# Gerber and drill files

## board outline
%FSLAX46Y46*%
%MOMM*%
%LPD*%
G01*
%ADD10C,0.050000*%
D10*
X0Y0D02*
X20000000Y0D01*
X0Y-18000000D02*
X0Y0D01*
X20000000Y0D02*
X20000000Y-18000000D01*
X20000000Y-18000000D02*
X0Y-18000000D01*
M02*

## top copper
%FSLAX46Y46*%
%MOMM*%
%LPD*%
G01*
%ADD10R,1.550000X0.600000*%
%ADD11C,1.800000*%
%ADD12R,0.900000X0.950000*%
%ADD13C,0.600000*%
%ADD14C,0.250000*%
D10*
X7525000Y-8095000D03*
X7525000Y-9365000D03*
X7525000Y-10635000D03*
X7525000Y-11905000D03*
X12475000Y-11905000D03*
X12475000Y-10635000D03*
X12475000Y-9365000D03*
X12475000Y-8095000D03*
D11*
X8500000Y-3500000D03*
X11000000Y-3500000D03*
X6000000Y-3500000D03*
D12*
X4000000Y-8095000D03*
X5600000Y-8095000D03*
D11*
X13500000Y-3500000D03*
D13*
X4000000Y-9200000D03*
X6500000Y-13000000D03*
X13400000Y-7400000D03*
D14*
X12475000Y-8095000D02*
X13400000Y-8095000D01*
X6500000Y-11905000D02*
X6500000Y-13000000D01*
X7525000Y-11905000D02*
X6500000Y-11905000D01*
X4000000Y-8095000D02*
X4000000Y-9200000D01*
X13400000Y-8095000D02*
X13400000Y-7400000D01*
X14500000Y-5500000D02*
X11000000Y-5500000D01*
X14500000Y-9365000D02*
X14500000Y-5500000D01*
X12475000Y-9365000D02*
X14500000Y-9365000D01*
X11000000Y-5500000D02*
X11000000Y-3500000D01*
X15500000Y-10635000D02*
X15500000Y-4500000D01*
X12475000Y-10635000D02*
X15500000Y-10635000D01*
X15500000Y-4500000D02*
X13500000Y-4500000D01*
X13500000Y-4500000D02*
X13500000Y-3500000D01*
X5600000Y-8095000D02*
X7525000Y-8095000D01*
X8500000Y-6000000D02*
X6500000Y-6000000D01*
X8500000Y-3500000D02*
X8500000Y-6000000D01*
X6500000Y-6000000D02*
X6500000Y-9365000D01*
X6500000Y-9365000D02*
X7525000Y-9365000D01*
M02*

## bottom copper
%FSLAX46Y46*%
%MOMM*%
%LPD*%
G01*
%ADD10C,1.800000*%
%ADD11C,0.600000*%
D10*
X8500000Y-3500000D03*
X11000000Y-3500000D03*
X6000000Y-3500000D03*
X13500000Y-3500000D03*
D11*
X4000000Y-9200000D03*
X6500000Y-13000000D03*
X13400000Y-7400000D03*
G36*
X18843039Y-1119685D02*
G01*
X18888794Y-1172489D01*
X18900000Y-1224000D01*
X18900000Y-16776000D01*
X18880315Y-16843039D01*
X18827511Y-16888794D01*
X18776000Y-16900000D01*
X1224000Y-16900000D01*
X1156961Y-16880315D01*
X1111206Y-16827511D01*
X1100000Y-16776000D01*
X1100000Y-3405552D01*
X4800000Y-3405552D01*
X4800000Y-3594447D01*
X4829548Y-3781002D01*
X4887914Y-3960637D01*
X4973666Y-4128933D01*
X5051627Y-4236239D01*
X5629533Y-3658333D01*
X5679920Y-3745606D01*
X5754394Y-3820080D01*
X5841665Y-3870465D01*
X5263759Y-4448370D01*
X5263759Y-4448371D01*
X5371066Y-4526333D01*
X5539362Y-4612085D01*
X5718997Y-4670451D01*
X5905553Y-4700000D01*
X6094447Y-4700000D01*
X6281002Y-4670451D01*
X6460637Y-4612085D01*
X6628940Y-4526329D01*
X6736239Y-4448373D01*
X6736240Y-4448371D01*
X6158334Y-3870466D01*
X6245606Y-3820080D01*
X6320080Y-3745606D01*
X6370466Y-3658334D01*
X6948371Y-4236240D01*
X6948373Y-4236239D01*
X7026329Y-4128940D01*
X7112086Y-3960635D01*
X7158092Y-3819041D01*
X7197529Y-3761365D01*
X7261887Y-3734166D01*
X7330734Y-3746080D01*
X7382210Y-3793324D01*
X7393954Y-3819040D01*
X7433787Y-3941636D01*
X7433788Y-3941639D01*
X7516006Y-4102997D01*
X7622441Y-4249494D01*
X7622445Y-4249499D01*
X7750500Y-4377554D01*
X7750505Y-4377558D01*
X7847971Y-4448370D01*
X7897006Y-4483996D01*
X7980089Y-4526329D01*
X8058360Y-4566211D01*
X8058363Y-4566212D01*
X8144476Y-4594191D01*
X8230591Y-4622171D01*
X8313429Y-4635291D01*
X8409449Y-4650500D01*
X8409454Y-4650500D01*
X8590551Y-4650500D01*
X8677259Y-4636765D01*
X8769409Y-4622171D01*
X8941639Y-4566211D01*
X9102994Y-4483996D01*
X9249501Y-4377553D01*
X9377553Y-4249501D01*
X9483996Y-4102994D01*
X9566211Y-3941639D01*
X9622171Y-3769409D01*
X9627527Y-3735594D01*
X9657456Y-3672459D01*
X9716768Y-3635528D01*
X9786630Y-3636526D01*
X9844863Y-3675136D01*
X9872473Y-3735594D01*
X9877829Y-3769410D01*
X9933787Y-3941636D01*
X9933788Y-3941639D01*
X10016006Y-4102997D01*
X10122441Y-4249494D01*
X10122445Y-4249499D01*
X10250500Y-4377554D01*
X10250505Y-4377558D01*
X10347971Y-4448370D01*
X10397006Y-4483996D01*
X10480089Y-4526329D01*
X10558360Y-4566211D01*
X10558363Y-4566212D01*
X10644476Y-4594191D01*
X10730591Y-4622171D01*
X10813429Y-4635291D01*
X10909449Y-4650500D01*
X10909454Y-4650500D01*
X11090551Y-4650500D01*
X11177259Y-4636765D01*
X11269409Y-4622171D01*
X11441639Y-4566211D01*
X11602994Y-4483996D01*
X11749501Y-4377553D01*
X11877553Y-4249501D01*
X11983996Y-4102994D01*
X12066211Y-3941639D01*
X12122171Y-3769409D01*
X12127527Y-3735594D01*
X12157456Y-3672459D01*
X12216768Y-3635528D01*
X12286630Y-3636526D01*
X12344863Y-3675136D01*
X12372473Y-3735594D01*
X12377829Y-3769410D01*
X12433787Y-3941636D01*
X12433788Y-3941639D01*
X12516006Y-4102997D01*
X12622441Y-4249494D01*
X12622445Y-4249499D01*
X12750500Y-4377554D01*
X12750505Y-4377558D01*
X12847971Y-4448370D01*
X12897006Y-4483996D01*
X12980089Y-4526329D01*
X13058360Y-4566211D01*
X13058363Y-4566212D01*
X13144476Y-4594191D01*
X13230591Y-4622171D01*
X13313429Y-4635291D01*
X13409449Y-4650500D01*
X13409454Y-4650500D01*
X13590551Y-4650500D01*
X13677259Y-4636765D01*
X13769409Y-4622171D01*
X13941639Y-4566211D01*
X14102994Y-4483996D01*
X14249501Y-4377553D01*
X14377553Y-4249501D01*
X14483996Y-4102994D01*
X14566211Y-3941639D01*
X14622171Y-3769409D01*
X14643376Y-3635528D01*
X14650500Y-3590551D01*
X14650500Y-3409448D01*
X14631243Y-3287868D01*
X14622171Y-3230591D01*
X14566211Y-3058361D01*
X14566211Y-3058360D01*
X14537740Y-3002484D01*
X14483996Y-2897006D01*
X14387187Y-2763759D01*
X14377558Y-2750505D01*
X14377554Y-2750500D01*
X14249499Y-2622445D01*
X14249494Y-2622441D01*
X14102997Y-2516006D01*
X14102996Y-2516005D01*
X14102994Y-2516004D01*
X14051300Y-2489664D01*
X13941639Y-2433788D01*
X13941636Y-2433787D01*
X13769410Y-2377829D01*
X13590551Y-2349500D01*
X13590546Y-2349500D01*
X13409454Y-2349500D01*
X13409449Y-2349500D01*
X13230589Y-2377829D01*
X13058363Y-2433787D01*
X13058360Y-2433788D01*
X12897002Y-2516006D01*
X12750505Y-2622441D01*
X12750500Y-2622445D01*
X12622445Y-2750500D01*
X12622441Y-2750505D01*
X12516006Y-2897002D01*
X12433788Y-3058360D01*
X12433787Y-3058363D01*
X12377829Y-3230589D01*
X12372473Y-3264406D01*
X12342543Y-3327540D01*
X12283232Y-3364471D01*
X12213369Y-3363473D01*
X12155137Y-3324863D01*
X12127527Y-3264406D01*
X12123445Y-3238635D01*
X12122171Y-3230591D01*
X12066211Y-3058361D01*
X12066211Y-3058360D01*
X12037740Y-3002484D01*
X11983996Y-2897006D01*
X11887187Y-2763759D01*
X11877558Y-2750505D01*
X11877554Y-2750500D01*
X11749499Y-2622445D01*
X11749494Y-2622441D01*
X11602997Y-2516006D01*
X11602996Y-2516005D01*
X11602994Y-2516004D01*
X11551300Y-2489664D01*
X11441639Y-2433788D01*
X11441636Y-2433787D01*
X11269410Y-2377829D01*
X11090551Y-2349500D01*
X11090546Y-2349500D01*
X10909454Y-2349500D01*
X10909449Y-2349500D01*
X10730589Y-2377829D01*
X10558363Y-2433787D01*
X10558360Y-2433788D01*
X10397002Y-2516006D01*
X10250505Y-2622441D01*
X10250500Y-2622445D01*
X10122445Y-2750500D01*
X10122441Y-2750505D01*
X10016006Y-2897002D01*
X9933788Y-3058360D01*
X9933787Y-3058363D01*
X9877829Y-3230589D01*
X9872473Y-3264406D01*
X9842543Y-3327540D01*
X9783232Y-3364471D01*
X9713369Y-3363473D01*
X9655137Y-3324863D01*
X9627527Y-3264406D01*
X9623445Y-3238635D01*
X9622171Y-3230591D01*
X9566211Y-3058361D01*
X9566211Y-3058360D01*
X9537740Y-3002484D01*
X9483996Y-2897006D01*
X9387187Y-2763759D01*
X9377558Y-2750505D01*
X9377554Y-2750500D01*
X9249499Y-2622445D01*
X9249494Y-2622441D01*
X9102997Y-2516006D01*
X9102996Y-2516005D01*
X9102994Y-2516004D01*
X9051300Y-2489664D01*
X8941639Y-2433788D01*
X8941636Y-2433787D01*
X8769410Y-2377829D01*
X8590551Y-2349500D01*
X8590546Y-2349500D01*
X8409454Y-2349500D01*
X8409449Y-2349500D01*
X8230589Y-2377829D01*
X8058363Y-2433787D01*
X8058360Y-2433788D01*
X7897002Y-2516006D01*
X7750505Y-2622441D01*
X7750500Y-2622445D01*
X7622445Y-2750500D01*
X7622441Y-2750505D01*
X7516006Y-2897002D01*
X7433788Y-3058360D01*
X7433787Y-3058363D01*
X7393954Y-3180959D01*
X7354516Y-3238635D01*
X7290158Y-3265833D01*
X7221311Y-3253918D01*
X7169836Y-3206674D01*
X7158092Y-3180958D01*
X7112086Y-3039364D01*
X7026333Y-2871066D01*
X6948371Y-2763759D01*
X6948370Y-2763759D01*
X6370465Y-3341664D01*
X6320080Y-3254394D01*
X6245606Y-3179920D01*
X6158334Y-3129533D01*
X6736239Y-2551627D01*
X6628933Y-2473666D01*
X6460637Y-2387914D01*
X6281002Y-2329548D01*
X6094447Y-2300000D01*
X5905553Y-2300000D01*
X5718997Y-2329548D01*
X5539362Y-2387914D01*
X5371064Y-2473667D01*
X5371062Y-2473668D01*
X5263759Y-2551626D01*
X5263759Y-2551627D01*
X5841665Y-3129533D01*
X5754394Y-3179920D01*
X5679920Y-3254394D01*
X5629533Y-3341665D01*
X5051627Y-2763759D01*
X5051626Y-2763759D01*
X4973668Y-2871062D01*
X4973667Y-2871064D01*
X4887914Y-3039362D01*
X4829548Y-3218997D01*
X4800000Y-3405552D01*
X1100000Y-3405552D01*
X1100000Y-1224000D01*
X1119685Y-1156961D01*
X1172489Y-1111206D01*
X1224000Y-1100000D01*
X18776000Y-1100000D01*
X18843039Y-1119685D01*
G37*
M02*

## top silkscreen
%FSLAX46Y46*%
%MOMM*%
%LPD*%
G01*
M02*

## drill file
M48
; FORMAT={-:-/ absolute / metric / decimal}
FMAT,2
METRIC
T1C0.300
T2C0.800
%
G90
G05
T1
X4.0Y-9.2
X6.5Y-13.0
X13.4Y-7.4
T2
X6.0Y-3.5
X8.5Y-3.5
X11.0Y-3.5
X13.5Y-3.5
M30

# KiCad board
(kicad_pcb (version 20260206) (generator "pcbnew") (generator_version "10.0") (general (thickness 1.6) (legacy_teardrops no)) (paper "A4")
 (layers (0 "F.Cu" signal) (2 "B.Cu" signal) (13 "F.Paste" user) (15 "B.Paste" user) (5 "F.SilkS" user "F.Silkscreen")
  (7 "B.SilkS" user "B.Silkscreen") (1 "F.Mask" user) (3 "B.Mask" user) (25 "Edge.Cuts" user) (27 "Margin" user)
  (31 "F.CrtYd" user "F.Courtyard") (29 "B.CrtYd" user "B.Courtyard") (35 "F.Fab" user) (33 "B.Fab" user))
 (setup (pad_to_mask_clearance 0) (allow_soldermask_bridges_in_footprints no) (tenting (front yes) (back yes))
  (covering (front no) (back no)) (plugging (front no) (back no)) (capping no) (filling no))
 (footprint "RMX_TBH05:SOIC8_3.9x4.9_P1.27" (layer "F.Cu") (at 10 10)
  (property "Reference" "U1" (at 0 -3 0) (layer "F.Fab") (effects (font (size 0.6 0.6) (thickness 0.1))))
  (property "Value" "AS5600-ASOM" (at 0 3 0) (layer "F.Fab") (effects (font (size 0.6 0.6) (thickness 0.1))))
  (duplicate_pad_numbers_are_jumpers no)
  (pad "1" smd rect (at -2.475 -1.905) (size 1.55 0.6) (layers "F.Cu" "F.Mask" "F.Paste") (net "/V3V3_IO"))
  (pad "2" smd rect (at -2.475 -0.635) (size 1.55 0.6) (layers "F.Cu" "F.Mask" "F.Paste") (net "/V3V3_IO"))
  (pad "3" smd rect (at -2.475 0.635) (size 1.55 0.6) (layers "F.Cu" "F.Mask" "F.Paste") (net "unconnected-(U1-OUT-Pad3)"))
  (pad "4" smd rect (at -2.475 1.905) (size 1.55 0.6) (layers "F.Cu" "F.Mask" "F.Paste") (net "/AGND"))
  (pad "5" smd rect (at 2.475 1.905) (size 1.55 0.6) (layers "F.Cu" "F.Mask" "F.Paste") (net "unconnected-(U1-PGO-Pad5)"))
  (pad "6" smd rect (at 2.475 0.635) (size 1.55 0.6) (layers "F.Cu" "F.Mask" "F.Paste") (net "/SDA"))
  (pad "7" smd rect (at 2.475 -0.635) (size 1.55 0.6) (layers "F.Cu" "F.Mask" "F.Paste") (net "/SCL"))
  (pad "8" smd rect (at 2.475 -1.905) (size 1.55 0.6) (layers "F.Cu" "F.Mask" "F.Paste") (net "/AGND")))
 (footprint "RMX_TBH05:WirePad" (layer "F.Cu") (at 8.5 3.5)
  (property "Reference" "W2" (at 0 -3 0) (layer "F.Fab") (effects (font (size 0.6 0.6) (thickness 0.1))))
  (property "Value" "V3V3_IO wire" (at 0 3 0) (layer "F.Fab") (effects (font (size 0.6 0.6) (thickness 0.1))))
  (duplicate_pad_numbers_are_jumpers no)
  (pad "1" thru_hole circle (at 0 0) (size 1.8 1.8) (drill 0.8) (layers "*.Cu" "*.Mask") (remove_unused_layers no) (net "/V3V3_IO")))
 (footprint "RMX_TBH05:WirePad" (layer "F.Cu") (at 11 3.5)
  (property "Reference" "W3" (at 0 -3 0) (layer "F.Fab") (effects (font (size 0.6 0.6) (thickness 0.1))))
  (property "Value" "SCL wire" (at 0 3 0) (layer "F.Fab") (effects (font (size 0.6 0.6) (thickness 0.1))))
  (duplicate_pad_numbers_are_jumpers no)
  (pad "1" thru_hole circle (at 0 0) (size 1.8 1.8) (drill 0.8) (layers "*.Cu" "*.Mask") (remove_unused_layers no) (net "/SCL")))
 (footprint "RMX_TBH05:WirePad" (layer "F.Cu") (at 6 3.5)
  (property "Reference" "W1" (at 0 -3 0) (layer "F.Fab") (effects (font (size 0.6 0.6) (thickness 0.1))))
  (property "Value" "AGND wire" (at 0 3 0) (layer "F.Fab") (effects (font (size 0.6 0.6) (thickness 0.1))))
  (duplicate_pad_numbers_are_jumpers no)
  (pad "1" thru_hole circle (at 0 0) (size 1.8 1.8) (drill 0.8) (layers "*.Cu" "*.Mask") (remove_unused_layers no) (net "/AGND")))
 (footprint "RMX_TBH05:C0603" (layer "F.Cu") (at 4.8 8.095)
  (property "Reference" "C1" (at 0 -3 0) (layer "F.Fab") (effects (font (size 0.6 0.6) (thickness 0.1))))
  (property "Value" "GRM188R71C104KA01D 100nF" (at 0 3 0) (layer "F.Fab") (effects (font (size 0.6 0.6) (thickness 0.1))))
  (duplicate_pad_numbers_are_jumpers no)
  (pad "1" smd rect (at -0.8 0) (size 0.9 0.95) (layers "F.Cu" "F.Mask" "F.Paste") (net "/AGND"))
  (pad "2" smd rect (at 0.8 0) (size 0.9 0.95) (layers "F.Cu" "F.Mask" "F.Paste") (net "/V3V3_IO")))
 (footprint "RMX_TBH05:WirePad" (layer "F.Cu") (at 13.5 3.5)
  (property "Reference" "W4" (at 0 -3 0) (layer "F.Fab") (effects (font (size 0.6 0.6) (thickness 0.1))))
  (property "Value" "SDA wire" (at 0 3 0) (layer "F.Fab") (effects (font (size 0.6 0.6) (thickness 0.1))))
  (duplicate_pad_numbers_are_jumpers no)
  (pad "1" thru_hole circle (at 0 0) (size 1.8 1.8) (drill 0.8) (layers "*.Cu" "*.Mask") (remove_unused_layers no) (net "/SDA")))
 (gr_line (start 0 0) (end 20 0) (stroke (width 0.05) (type default)) (layer "Edge.Cuts"))
 (gr_line (start 0 18) (end 0 0) (stroke (width 0.05) (type default)) (layer "Edge.Cuts"))
 (gr_line (start 20 0) (end 20 18) (stroke (width 0.05) (type default)) (layer "Edge.Cuts"))
 (gr_line (start 20 18) (end 0 18) (stroke (width 0.05) (type default)) (layer "Edge.Cuts"))
 (segment (start 12.475 8.095) (end 13.4 8.095) (width 0.25) (layer "F.Cu") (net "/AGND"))
 (segment (start 6.5 11.905) (end 6.5 13) (width 0.25) (layer "F.Cu") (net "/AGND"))
 (segment (start 7.525 11.905) (end 6.5 11.905) (width 0.25) (layer "F.Cu") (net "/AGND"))
 (segment (start 4 8.095) (end 4 9.2) (width 0.25) (layer "F.Cu") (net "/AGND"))
 (segment (start 13.4 8.095) (end 13.4 7.4) (width 0.25) (layer "F.Cu") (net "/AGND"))
 (via (at 4 9.2) (size 0.6) (drill 0.3) (layers "F.Cu" "B.Cu") (capping no) (covering (front no) (back no)) (plugging (front no) (back no))
  (filling no) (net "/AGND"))
 (via (at 6.5 13) (size 0.6) (drill 0.3) (layers "F.Cu" "B.Cu") (capping no) (covering (front no) (back no)) (plugging (front no) (back no))
  (filling no) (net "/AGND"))
 (via (at 13.4 7.4) (size 0.6) (drill 0.3) (layers "F.Cu" "B.Cu") (capping no) (covering (front no) (back no))
  (plugging (front no) (back no)) (filling no) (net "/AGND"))
 (segment (start 14.5 5.5) (end 11 5.5) (width 0.25) (layer "F.Cu") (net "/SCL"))
 (segment (start 14.5 9.365) (end 14.5 5.5) (width 0.25) (layer "F.Cu") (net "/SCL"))
 (segment (start 12.475 9.365) (end 14.5 9.365) (width 0.25) (layer "F.Cu") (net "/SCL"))
 (segment (start 11 5.5) (end 11 3.5) (width 0.25) (layer "F.Cu") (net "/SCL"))
 (segment (start 15.5 10.635) (end 15.5 4.5) (width 0.25) (layer "F.Cu") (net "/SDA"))
 (segment (start 12.475 10.635) (end 15.5 10.635) (width 0.25) (layer "F.Cu") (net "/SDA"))
 (segment (start 15.5 4.5) (end 13.5 4.5) (width 0.25) (layer "F.Cu") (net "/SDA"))
 (segment (start 13.5 4.5) (end 13.5 3.5) (width 0.25) (layer "F.Cu") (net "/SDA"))
 (segment (start 5.6 8.095) (end 7.525 8.095) (width 0.25) (layer "F.Cu") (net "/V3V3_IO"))
 (segment (start 8.5 6) (end 6.5 6) (width 0.25) (layer "F.Cu") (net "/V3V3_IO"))
 (segment (start 8.5 3.5) (end 8.5 6) (width 0.25) (layer "F.Cu") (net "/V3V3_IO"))
 (segment (start 6.5 6) (end 6.5 9.365) (width 0.25) (layer "F.Cu") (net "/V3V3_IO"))
 (segment (start 6.5 9.365) (end 7.525 9.365) (width 0.25) (layer "F.Cu") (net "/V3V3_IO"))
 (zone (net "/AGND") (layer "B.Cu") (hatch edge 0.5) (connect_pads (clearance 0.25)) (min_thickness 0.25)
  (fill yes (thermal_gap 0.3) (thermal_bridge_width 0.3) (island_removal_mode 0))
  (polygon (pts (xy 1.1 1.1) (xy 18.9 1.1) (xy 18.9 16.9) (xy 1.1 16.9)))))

